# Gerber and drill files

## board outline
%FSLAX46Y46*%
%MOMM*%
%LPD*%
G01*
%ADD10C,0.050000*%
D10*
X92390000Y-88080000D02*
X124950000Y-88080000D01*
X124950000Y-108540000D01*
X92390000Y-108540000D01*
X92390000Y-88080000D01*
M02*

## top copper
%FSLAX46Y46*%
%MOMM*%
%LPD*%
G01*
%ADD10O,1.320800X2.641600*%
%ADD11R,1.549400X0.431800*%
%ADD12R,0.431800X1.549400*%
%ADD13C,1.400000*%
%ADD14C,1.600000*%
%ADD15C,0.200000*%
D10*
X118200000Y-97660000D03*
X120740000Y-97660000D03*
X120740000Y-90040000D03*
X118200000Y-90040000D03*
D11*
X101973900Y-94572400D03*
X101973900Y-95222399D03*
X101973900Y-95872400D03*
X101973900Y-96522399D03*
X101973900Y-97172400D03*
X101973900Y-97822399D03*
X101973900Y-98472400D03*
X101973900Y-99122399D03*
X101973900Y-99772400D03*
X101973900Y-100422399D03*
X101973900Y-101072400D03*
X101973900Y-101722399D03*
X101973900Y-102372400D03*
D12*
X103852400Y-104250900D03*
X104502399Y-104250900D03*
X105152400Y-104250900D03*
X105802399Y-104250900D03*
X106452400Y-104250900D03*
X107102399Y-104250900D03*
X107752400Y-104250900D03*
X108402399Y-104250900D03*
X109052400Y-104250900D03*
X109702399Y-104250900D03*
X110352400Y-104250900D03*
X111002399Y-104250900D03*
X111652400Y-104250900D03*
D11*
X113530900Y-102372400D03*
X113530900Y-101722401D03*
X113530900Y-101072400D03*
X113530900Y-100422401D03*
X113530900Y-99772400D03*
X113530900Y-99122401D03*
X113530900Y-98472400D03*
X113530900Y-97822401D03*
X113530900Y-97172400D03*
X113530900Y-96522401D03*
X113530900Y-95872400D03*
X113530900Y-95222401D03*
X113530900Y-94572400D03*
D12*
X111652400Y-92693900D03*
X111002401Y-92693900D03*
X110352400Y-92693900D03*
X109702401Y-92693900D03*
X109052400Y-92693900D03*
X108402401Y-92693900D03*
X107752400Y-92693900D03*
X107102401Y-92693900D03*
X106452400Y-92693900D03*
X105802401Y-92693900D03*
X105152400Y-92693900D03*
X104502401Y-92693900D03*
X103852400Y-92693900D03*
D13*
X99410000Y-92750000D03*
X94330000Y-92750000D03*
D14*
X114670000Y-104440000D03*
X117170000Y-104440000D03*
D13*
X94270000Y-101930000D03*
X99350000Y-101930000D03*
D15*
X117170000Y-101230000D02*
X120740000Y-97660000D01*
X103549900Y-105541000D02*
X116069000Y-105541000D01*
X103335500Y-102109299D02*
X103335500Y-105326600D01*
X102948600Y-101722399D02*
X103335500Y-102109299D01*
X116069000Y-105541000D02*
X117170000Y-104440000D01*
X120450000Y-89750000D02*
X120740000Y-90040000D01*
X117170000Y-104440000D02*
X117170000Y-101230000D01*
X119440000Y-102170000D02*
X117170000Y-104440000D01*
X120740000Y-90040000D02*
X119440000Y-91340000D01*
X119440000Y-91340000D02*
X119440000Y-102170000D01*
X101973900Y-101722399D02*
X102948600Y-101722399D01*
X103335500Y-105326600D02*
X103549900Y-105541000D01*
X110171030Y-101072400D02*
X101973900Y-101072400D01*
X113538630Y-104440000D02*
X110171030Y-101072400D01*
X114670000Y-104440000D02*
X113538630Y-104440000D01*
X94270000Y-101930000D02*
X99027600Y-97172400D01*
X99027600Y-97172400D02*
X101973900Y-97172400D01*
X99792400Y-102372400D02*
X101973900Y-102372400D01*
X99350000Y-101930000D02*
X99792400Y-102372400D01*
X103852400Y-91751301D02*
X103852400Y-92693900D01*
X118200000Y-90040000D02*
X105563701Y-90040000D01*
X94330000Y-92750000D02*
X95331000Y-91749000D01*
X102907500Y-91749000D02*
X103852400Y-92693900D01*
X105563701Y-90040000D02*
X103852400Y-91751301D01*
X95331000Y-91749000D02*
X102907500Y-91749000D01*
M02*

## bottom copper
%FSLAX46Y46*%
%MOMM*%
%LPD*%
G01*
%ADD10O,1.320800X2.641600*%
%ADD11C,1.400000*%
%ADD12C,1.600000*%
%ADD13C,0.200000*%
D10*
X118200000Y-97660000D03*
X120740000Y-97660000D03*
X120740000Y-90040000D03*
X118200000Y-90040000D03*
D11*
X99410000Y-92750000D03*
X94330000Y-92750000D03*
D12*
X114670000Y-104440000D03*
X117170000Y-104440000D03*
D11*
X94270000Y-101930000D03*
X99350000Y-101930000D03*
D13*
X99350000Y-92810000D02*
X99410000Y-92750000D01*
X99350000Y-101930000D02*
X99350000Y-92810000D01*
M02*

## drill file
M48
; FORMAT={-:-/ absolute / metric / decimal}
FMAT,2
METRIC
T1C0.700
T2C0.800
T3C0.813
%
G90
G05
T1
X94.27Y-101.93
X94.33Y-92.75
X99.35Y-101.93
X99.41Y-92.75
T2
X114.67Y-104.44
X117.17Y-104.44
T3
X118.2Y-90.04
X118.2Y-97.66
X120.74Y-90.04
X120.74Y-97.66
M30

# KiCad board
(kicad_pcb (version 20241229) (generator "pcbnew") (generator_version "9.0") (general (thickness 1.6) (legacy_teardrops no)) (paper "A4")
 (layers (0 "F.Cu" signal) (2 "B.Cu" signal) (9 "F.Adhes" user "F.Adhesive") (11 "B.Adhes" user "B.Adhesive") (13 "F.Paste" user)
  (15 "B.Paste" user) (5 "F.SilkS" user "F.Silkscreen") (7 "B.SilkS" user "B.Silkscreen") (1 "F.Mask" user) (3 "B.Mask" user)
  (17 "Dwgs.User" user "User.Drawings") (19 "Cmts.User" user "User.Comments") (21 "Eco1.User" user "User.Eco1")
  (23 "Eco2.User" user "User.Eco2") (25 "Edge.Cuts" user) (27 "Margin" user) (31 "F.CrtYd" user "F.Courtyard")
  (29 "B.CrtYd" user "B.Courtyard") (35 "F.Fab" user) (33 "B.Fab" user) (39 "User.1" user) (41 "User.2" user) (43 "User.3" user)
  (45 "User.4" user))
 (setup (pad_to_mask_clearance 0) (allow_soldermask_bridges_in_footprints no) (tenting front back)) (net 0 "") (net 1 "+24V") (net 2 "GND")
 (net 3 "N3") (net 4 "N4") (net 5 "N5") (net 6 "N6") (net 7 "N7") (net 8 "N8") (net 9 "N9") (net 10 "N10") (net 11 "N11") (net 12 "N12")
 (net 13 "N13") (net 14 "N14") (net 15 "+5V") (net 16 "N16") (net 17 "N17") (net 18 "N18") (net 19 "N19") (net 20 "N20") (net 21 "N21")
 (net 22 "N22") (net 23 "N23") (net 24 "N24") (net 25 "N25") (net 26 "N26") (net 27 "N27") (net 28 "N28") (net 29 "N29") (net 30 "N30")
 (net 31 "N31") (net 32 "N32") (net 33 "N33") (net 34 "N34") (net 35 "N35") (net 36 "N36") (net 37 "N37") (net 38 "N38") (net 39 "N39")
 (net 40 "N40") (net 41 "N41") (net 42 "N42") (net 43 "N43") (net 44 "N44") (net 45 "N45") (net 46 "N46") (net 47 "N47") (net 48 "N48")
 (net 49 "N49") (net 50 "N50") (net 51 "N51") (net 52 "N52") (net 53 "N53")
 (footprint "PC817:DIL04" (layer "F.Cu") (at 119.47 93.85)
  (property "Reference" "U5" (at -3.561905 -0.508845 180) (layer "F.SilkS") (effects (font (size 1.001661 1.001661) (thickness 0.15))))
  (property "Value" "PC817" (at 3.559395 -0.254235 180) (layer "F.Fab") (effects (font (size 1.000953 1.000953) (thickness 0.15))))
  (pad "1" thru_hole oval (at -1.27 3.81) (size 1.3208 2.6416) (drill 0.8128) (layers "*.Cu" "*.Mask") (remove_unused_layers no)
   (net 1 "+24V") (solder_mask_margin 0.102))
  (pad "2" thru_hole oval (at 1.27 3.81) (size 1.3208 2.6416) (drill 0.8128) (layers "*.Cu" "*.Mask") (remove_unused_layers no)
   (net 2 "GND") (solder_mask_margin 0.102))
  (pad "3" thru_hole oval (at 1.27 -3.81) (size 1.3208 2.6416) (drill 0.8128) (layers "*.Cu" "*.Mask") (remove_unused_layers no)
   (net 2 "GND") (solder_mask_margin 0.102))
  (pad "4" thru_hole oval (at -1.27 -3.81) (size 1.3208 2.6416) (drill 0.8128) (layers "*.Cu" "*.Mask") (remove_unused_layers no)
   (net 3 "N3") (solder_mask_margin 0.102)))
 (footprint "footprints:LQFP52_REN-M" (layer "F.Cu") (at 107.7524 98.4724)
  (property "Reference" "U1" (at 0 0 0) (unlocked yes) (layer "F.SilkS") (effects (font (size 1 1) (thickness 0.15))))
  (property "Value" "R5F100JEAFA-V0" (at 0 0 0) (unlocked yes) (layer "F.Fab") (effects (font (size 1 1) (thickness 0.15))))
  (pad "1" smd rect (at -5.7785 -3.9 90) (size 0.4318 1.5494) (layers "F.Cu" "F.Mask" "F.Paste") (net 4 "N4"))
  (pad "2" smd rect (at -5.7785 -3.250001 90) (size 0.4318 1.5494) (layers "F.Cu" "F.Mask" "F.Paste") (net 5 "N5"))
  (pad "3" smd rect (at -5.7785 -2.6 90) (size 0.4318 1.5494) (layers "F.Cu" "F.Mask" "F.Paste") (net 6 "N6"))
  (pad "4" smd rect (at -5.7785 -1.950001 90) (size 0.4318 1.5494) (layers "F.Cu" "F.Mask" "F.Paste") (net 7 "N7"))
  (pad "5" smd rect (at -5.7785 -1.3 90) (size 0.4318 1.5494) (layers "F.Cu" "F.Mask" "F.Paste") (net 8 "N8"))
  (pad "6" smd rect (at -5.7785 -0.650001 90) (size 0.4318 1.5494) (layers "F.Cu" "F.Mask" "F.Paste") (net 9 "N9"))
  (pad "7" smd rect (at -5.7785 0 90) (size 0.4318 1.5494) (layers "F.Cu" "F.Mask" "F.Paste") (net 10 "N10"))
  (pad "8" smd rect (at -5.7785 0.649999 90) (size 0.4318 1.5494) (layers "F.Cu" "F.Mask" "F.Paste") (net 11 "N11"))
  (pad "9" smd rect (at -5.7785 1.3 90) (size 0.4318 1.5494) (layers "F.Cu" "F.Mask" "F.Paste") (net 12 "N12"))
  (pad "10" smd rect (at -5.7785 1.949999 90) (size 0.4318 1.5494) (layers "F.Cu" "F.Mask" "F.Paste") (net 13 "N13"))
  (pad "11" smd rect (at -5.7785 2.6 90) (size 0.4318 1.5494) (layers "F.Cu" "F.Mask" "F.Paste") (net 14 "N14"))
  (pad "12" smd rect (at -5.7785 3.249999 90) (size 0.4318 1.5494) (layers "F.Cu" "F.Mask" "F.Paste") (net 2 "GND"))
  (pad "13" smd rect (at -5.7785 3.9 90) (size 0.4318 1.5494) (layers "F.Cu" "F.Mask" "F.Paste") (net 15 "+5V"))
  (pad "14" smd rect (at -3.9 5.7785) (size 0.4318 1.5494) (layers "F.Cu" "F.Mask" "F.Paste") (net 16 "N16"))
  (pad "15" smd rect (at -3.250001 5.7785) (size 0.4318 1.5494) (layers "F.Cu" "F.Mask" "F.Paste") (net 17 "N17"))
  (pad "16" smd rect (at -2.6 5.7785) (size 0.4318 1.5494) (layers "F.Cu" "F.Mask" "F.Paste") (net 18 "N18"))
  (pad "17" smd rect (at -1.950001 5.7785) (size 0.4318 1.5494) (layers "F.Cu" "F.Mask" "F.Paste") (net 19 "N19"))
  (pad "18" smd rect (at -1.3 5.7785) (size 0.4318 1.5494) (layers "F.Cu" "F.Mask" "F.Paste") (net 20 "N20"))
  (pad "19" smd rect (at -0.650001 5.7785) (size 0.4318 1.5494) (layers "F.Cu" "F.Mask" "F.Paste") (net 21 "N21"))
  (pad "20" smd rect (at 0 5.7785) (size 0.4318 1.5494) (layers "F.Cu" "F.Mask" "F.Paste") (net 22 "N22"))
  (pad "21" smd rect (at 0.649999 5.7785) (size 0.4318 1.5494) (layers "F.Cu" "F.Mask" "F.Paste") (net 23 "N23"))
  (pad "22" smd rect (at 1.3 5.7785) (size 0.4318 1.5494) (layers "F.Cu" "F.Mask" "F.Paste") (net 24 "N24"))
  (pad "23" smd rect (at 1.949999 5.7785) (size 0.4318 1.5494) (layers "F.Cu" "F.Mask" "F.Paste") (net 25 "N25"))
  (pad "24" smd rect (at 2.6 5.7785) (size 0.4318 1.5494) (layers "F.Cu" "F.Mask" "F.Paste") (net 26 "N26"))
  (pad "25" smd rect (at 3.249999 5.7785) (size 0.4318 1.5494) (layers "F.Cu" "F.Mask" "F.Paste") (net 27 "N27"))
  (pad "26" smd rect (at 3.9 5.7785) (size 0.4318 1.5494) (layers "F.Cu" "F.Mask" "F.Paste") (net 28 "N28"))
  (pad "27" smd rect (at 5.7785 3.9 90) (size 0.4318 1.5494) (layers "F.Cu" "F.Mask" "F.Paste") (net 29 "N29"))
  (pad "28" smd rect (at 5.7785 3.250001 90) (size 0.4318 1.5494) (layers "F.Cu" "F.Mask" "F.Paste") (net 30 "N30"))
  (pad "29" smd rect (at 5.7785 2.6 90) (size 0.4318 1.5494) (layers "F.Cu" "F.Mask" "F.Paste") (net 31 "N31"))
  (pad "30" smd rect (at 5.7785 1.950001 90) (size 0.4318 1.5494) (layers "F.Cu" "F.Mask" "F.Paste") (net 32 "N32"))
  (pad "31" smd rect (at 5.7785 1.3 90) (size 0.4318 1.5494) (layers "F.Cu" "F.Mask" "F.Paste") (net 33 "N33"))
  (pad "32" smd rect (at 5.7785 0.650001 90) (size 0.4318 1.5494) (layers "F.Cu" "F.Mask" "F.Paste") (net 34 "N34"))
  (pad "33" smd rect (at 5.7785 0 90) (size 0.4318 1.5494) (layers "F.Cu" "F.Mask" "F.Paste") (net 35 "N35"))
  (pad "34" smd rect (at 5.7785 -0.649999 90) (size 0.4318 1.5494) (layers "F.Cu" "F.Mask" "F.Paste") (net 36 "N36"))
  (pad "35" smd rect (at 5.7785 -1.3 90) (size 0.4318 1.5494) (layers "F.Cu" "F.Mask" "F.Paste") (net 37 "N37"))
  (pad "36" smd rect (at 5.7785 -1.949999 90) (size 0.4318 1.5494) (layers "F.Cu" "F.Mask" "F.Paste") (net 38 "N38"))
  (pad "37" smd rect (at 5.7785 -2.6 90) (size 0.4318 1.5494) (layers "F.Cu" "F.Mask" "F.Paste") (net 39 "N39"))
  (pad "38" smd rect (at 5.7785 -3.249999 90) (size 0.4318 1.5494) (layers "F.Cu" "F.Mask" "F.Paste") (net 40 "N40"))
  (pad "39" smd rect (at 5.7785 -3.9 90) (size 0.4318 1.5494) (layers "F.Cu" "F.Mask" "F.Paste") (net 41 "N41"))
  (pad "40" smd rect (at 3.9 -5.7785) (size 0.4318 1.5494) (layers "F.Cu" "F.Mask" "F.Paste") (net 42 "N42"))
  (pad "41" smd rect (at 3.250001 -5.7785) (size 0.4318 1.5494) (layers "F.Cu" "F.Mask" "F.Paste") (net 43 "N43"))
  (pad "42" smd rect (at 2.6 -5.7785) (size 0.4318 1.5494) (layers "F.Cu" "F.Mask" "F.Paste") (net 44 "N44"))
  (pad "43" smd rect (at 1.950001 -5.7785) (size 0.4318 1.5494) (layers "F.Cu" "F.Mask" "F.Paste") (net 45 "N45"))
  (pad "44" smd rect (at 1.3 -5.7785) (size 0.4318 1.5494) (layers "F.Cu" "F.Mask" "F.Paste") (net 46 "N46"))
  (pad "45" smd rect (at 0.650001 -5.7785) (size 0.4318 1.5494) (layers "F.Cu" "F.Mask" "F.Paste") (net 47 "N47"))
  (pad "46" smd rect (at 0 -5.7785) (size 0.4318 1.5494) (layers "F.Cu" "F.Mask" "F.Paste") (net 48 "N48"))
  (pad "47" smd rect (at -0.649999 -5.7785) (size 0.4318 1.5494) (layers "F.Cu" "F.Mask" "F.Paste") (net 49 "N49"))
  (pad "48" smd rect (at -1.3 -5.7785) (size 0.4318 1.5494) (layers "F.Cu" "F.Mask" "F.Paste") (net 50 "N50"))
  (pad "49" smd rect (at -1.949999 -5.7785) (size 0.4318 1.5494) (layers "F.Cu" "F.Mask" "F.Paste") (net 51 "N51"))
  (pad "50" smd rect (at -2.6 -5.7785) (size 0.4318 1.5494) (layers "F.Cu" "F.Mask" "F.Paste") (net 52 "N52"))
  (pad "51" smd rect (at -3.249999 -5.7785) (size 0.4318 1.5494) (layers "F.Cu" "F.Mask" "F.Paste") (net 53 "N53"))
  (pad "52" smd rect (at -3.9 -5.7785) (size 0.4318 1.5494) (layers "F.Cu" "F.Mask" "F.Paste") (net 3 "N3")))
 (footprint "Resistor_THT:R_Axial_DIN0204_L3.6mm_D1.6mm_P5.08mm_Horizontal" (layer "F.Cu") (at 99.41 92.75 180)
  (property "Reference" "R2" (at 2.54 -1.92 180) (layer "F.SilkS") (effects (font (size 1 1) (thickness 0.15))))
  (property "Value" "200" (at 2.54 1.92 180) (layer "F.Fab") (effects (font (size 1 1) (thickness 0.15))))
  (pad "1" thru_hole circle (at 0 0 180) (size 1.4 1.4) (drill 0.7) (layers "*.Cu" "*.Mask") (remove_unused_layers no) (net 15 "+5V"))
  (pad "2" thru_hole circle (at 5.08 0 180) (size 1.4 1.4) (drill 0.7) (layers "*.Cu" "*.Mask") (remove_unused_layers no) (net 3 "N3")))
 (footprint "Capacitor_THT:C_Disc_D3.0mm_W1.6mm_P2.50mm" (layer "F.Cu") (at 114.67 104.44)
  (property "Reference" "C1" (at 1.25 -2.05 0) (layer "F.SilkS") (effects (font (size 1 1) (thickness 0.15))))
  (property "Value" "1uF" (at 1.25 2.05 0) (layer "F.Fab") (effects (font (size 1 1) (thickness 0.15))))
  (pad "1" thru_hole circle (at 0 0) (size 1.6 1.6) (drill 0.8) (layers "*.Cu" "*.Mask") (remove_unused_layers no) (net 14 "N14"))
  (pad "2" thru_hole circle (at 2.5 0) (size 1.6 1.6) (drill 0.8) (layers "*.Cu" "*.Mask") (remove_unused_layers no) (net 2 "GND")))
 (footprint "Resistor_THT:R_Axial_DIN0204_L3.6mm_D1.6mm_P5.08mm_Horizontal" (layer "F.Cu") (at 94.27 101.93)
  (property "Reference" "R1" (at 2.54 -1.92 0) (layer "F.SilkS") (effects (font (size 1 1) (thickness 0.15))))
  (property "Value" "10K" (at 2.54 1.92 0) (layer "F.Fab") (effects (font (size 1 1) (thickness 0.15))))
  (pad "1" thru_hole circle (at 0 0) (size 1.4 1.4) (drill 0.7) (layers "*.Cu" "*.Mask") (remove_unused_layers no) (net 8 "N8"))
  (pad "2" thru_hole circle (at 5.08 0) (size 1.4 1.4) (drill 0.7) (layers "*.Cu" "*.Mask") (remove_unused_layers no) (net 15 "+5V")))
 (gr_rect (start 92.39 88.08) (end 124.95 108.54) (stroke (width 0.05) (type default)) (fill no) (layer "Edge.Cuts"))
 (segment (start 117.17 101.23) (end 120.74 97.66) (width 0.2) (layer "F.Cu") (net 2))
 (segment (start 103.5499 105.541) (end 116.069 105.541) (width 0.2) (layer "F.Cu") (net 2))
 (segment (start 103.3355 102.109299) (end 103.3355 105.3266) (width 0.2) (layer "F.Cu") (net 2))
 (segment (start 102.9486 101.722399) (end 103.3355 102.109299) (width 0.2) (layer "F.Cu") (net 2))
 (segment (start 116.069 105.541) (end 117.17 104.44) (width 0.2) (layer "F.Cu") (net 2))
 (segment (start 120.45 89.75) (end 120.74 90.04) (width 0.2) (layer "F.Cu") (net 2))
 (segment (start 117.17 104.44) (end 117.17 101.23) (width 0.2) (layer "F.Cu") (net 2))
 (segment (start 119.44 102.17) (end 117.17 104.44) (width 0.2) (layer "F.Cu") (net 2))
 (segment (start 120.74 90.04) (end 119.44 91.34) (width 0.2) (layer "F.Cu") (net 2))
 (segment (start 119.44 91.34) (end 119.44 102.17) (width 0.2) (layer "F.Cu") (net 2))
 (segment (start 101.9739 101.722399) (end 102.9486 101.722399) (width 0.2) (layer "F.Cu") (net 2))
 (segment (start 103.3355 105.3266) (end 103.5499 105.541) (width 0.2) (layer "F.Cu") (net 2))
 (segment (start 110.17103 101.0724) (end 101.9739 101.0724) (width 0.2) (layer "F.Cu") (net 14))
 (segment (start 113.53863 104.44) (end 110.17103 101.0724) (width 0.2) (layer "F.Cu") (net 14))
 (segment (start 114.67 104.44) (end 113.53863 104.44) (width 0.2) (layer "F.Cu") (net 14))
 (segment (start 94.27 101.93) (end 99.0276 97.1724) (width 0.2) (layer "F.Cu") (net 8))
 (segment (start 99.0276 97.1724) (end 101.9739 97.1724) (width 0.2) (layer "F.Cu") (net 8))
 (segment (start 99.7924 102.3724) (end 101.9739 102.3724) (width 0.2) (layer "F.Cu") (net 15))
 (segment (start 99.35 101.93) (end 99.7924 102.3724) (width 0.2) (layer "F.Cu") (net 15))
 (segment (start 99.35 92.81) (end 99.41 92.75) (width 0.2) (layer "B.Cu") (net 15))
 (segment (start 99.35 101.93) (end 99.35 92.81) (width 0.2) (layer "B.Cu") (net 15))
 (segment (start 103.8524 91.751301) (end 103.8524 92.6939) (width 0.2) (layer "F.Cu") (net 3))
 (segment (start 118.2 90.04) (end 105.563701 90.04) (width 0.2) (layer "F.Cu") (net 3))
 (segment (start 94.33 92.75) (end 95.331 91.749) (width 0.2) (layer "F.Cu") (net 3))
 (segment (start 102.9075 91.749) (end 103.8524 92.6939) (width 0.2) (layer "F.Cu") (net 3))
 (segment (start 105.563701 90.04) (end 103.8524 91.751301) (width 0.2) (layer "F.Cu") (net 3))
 (segment (start 95.331 91.749) (end 102.9075 91.749) (width 0.2) (layer "F.Cu") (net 3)))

